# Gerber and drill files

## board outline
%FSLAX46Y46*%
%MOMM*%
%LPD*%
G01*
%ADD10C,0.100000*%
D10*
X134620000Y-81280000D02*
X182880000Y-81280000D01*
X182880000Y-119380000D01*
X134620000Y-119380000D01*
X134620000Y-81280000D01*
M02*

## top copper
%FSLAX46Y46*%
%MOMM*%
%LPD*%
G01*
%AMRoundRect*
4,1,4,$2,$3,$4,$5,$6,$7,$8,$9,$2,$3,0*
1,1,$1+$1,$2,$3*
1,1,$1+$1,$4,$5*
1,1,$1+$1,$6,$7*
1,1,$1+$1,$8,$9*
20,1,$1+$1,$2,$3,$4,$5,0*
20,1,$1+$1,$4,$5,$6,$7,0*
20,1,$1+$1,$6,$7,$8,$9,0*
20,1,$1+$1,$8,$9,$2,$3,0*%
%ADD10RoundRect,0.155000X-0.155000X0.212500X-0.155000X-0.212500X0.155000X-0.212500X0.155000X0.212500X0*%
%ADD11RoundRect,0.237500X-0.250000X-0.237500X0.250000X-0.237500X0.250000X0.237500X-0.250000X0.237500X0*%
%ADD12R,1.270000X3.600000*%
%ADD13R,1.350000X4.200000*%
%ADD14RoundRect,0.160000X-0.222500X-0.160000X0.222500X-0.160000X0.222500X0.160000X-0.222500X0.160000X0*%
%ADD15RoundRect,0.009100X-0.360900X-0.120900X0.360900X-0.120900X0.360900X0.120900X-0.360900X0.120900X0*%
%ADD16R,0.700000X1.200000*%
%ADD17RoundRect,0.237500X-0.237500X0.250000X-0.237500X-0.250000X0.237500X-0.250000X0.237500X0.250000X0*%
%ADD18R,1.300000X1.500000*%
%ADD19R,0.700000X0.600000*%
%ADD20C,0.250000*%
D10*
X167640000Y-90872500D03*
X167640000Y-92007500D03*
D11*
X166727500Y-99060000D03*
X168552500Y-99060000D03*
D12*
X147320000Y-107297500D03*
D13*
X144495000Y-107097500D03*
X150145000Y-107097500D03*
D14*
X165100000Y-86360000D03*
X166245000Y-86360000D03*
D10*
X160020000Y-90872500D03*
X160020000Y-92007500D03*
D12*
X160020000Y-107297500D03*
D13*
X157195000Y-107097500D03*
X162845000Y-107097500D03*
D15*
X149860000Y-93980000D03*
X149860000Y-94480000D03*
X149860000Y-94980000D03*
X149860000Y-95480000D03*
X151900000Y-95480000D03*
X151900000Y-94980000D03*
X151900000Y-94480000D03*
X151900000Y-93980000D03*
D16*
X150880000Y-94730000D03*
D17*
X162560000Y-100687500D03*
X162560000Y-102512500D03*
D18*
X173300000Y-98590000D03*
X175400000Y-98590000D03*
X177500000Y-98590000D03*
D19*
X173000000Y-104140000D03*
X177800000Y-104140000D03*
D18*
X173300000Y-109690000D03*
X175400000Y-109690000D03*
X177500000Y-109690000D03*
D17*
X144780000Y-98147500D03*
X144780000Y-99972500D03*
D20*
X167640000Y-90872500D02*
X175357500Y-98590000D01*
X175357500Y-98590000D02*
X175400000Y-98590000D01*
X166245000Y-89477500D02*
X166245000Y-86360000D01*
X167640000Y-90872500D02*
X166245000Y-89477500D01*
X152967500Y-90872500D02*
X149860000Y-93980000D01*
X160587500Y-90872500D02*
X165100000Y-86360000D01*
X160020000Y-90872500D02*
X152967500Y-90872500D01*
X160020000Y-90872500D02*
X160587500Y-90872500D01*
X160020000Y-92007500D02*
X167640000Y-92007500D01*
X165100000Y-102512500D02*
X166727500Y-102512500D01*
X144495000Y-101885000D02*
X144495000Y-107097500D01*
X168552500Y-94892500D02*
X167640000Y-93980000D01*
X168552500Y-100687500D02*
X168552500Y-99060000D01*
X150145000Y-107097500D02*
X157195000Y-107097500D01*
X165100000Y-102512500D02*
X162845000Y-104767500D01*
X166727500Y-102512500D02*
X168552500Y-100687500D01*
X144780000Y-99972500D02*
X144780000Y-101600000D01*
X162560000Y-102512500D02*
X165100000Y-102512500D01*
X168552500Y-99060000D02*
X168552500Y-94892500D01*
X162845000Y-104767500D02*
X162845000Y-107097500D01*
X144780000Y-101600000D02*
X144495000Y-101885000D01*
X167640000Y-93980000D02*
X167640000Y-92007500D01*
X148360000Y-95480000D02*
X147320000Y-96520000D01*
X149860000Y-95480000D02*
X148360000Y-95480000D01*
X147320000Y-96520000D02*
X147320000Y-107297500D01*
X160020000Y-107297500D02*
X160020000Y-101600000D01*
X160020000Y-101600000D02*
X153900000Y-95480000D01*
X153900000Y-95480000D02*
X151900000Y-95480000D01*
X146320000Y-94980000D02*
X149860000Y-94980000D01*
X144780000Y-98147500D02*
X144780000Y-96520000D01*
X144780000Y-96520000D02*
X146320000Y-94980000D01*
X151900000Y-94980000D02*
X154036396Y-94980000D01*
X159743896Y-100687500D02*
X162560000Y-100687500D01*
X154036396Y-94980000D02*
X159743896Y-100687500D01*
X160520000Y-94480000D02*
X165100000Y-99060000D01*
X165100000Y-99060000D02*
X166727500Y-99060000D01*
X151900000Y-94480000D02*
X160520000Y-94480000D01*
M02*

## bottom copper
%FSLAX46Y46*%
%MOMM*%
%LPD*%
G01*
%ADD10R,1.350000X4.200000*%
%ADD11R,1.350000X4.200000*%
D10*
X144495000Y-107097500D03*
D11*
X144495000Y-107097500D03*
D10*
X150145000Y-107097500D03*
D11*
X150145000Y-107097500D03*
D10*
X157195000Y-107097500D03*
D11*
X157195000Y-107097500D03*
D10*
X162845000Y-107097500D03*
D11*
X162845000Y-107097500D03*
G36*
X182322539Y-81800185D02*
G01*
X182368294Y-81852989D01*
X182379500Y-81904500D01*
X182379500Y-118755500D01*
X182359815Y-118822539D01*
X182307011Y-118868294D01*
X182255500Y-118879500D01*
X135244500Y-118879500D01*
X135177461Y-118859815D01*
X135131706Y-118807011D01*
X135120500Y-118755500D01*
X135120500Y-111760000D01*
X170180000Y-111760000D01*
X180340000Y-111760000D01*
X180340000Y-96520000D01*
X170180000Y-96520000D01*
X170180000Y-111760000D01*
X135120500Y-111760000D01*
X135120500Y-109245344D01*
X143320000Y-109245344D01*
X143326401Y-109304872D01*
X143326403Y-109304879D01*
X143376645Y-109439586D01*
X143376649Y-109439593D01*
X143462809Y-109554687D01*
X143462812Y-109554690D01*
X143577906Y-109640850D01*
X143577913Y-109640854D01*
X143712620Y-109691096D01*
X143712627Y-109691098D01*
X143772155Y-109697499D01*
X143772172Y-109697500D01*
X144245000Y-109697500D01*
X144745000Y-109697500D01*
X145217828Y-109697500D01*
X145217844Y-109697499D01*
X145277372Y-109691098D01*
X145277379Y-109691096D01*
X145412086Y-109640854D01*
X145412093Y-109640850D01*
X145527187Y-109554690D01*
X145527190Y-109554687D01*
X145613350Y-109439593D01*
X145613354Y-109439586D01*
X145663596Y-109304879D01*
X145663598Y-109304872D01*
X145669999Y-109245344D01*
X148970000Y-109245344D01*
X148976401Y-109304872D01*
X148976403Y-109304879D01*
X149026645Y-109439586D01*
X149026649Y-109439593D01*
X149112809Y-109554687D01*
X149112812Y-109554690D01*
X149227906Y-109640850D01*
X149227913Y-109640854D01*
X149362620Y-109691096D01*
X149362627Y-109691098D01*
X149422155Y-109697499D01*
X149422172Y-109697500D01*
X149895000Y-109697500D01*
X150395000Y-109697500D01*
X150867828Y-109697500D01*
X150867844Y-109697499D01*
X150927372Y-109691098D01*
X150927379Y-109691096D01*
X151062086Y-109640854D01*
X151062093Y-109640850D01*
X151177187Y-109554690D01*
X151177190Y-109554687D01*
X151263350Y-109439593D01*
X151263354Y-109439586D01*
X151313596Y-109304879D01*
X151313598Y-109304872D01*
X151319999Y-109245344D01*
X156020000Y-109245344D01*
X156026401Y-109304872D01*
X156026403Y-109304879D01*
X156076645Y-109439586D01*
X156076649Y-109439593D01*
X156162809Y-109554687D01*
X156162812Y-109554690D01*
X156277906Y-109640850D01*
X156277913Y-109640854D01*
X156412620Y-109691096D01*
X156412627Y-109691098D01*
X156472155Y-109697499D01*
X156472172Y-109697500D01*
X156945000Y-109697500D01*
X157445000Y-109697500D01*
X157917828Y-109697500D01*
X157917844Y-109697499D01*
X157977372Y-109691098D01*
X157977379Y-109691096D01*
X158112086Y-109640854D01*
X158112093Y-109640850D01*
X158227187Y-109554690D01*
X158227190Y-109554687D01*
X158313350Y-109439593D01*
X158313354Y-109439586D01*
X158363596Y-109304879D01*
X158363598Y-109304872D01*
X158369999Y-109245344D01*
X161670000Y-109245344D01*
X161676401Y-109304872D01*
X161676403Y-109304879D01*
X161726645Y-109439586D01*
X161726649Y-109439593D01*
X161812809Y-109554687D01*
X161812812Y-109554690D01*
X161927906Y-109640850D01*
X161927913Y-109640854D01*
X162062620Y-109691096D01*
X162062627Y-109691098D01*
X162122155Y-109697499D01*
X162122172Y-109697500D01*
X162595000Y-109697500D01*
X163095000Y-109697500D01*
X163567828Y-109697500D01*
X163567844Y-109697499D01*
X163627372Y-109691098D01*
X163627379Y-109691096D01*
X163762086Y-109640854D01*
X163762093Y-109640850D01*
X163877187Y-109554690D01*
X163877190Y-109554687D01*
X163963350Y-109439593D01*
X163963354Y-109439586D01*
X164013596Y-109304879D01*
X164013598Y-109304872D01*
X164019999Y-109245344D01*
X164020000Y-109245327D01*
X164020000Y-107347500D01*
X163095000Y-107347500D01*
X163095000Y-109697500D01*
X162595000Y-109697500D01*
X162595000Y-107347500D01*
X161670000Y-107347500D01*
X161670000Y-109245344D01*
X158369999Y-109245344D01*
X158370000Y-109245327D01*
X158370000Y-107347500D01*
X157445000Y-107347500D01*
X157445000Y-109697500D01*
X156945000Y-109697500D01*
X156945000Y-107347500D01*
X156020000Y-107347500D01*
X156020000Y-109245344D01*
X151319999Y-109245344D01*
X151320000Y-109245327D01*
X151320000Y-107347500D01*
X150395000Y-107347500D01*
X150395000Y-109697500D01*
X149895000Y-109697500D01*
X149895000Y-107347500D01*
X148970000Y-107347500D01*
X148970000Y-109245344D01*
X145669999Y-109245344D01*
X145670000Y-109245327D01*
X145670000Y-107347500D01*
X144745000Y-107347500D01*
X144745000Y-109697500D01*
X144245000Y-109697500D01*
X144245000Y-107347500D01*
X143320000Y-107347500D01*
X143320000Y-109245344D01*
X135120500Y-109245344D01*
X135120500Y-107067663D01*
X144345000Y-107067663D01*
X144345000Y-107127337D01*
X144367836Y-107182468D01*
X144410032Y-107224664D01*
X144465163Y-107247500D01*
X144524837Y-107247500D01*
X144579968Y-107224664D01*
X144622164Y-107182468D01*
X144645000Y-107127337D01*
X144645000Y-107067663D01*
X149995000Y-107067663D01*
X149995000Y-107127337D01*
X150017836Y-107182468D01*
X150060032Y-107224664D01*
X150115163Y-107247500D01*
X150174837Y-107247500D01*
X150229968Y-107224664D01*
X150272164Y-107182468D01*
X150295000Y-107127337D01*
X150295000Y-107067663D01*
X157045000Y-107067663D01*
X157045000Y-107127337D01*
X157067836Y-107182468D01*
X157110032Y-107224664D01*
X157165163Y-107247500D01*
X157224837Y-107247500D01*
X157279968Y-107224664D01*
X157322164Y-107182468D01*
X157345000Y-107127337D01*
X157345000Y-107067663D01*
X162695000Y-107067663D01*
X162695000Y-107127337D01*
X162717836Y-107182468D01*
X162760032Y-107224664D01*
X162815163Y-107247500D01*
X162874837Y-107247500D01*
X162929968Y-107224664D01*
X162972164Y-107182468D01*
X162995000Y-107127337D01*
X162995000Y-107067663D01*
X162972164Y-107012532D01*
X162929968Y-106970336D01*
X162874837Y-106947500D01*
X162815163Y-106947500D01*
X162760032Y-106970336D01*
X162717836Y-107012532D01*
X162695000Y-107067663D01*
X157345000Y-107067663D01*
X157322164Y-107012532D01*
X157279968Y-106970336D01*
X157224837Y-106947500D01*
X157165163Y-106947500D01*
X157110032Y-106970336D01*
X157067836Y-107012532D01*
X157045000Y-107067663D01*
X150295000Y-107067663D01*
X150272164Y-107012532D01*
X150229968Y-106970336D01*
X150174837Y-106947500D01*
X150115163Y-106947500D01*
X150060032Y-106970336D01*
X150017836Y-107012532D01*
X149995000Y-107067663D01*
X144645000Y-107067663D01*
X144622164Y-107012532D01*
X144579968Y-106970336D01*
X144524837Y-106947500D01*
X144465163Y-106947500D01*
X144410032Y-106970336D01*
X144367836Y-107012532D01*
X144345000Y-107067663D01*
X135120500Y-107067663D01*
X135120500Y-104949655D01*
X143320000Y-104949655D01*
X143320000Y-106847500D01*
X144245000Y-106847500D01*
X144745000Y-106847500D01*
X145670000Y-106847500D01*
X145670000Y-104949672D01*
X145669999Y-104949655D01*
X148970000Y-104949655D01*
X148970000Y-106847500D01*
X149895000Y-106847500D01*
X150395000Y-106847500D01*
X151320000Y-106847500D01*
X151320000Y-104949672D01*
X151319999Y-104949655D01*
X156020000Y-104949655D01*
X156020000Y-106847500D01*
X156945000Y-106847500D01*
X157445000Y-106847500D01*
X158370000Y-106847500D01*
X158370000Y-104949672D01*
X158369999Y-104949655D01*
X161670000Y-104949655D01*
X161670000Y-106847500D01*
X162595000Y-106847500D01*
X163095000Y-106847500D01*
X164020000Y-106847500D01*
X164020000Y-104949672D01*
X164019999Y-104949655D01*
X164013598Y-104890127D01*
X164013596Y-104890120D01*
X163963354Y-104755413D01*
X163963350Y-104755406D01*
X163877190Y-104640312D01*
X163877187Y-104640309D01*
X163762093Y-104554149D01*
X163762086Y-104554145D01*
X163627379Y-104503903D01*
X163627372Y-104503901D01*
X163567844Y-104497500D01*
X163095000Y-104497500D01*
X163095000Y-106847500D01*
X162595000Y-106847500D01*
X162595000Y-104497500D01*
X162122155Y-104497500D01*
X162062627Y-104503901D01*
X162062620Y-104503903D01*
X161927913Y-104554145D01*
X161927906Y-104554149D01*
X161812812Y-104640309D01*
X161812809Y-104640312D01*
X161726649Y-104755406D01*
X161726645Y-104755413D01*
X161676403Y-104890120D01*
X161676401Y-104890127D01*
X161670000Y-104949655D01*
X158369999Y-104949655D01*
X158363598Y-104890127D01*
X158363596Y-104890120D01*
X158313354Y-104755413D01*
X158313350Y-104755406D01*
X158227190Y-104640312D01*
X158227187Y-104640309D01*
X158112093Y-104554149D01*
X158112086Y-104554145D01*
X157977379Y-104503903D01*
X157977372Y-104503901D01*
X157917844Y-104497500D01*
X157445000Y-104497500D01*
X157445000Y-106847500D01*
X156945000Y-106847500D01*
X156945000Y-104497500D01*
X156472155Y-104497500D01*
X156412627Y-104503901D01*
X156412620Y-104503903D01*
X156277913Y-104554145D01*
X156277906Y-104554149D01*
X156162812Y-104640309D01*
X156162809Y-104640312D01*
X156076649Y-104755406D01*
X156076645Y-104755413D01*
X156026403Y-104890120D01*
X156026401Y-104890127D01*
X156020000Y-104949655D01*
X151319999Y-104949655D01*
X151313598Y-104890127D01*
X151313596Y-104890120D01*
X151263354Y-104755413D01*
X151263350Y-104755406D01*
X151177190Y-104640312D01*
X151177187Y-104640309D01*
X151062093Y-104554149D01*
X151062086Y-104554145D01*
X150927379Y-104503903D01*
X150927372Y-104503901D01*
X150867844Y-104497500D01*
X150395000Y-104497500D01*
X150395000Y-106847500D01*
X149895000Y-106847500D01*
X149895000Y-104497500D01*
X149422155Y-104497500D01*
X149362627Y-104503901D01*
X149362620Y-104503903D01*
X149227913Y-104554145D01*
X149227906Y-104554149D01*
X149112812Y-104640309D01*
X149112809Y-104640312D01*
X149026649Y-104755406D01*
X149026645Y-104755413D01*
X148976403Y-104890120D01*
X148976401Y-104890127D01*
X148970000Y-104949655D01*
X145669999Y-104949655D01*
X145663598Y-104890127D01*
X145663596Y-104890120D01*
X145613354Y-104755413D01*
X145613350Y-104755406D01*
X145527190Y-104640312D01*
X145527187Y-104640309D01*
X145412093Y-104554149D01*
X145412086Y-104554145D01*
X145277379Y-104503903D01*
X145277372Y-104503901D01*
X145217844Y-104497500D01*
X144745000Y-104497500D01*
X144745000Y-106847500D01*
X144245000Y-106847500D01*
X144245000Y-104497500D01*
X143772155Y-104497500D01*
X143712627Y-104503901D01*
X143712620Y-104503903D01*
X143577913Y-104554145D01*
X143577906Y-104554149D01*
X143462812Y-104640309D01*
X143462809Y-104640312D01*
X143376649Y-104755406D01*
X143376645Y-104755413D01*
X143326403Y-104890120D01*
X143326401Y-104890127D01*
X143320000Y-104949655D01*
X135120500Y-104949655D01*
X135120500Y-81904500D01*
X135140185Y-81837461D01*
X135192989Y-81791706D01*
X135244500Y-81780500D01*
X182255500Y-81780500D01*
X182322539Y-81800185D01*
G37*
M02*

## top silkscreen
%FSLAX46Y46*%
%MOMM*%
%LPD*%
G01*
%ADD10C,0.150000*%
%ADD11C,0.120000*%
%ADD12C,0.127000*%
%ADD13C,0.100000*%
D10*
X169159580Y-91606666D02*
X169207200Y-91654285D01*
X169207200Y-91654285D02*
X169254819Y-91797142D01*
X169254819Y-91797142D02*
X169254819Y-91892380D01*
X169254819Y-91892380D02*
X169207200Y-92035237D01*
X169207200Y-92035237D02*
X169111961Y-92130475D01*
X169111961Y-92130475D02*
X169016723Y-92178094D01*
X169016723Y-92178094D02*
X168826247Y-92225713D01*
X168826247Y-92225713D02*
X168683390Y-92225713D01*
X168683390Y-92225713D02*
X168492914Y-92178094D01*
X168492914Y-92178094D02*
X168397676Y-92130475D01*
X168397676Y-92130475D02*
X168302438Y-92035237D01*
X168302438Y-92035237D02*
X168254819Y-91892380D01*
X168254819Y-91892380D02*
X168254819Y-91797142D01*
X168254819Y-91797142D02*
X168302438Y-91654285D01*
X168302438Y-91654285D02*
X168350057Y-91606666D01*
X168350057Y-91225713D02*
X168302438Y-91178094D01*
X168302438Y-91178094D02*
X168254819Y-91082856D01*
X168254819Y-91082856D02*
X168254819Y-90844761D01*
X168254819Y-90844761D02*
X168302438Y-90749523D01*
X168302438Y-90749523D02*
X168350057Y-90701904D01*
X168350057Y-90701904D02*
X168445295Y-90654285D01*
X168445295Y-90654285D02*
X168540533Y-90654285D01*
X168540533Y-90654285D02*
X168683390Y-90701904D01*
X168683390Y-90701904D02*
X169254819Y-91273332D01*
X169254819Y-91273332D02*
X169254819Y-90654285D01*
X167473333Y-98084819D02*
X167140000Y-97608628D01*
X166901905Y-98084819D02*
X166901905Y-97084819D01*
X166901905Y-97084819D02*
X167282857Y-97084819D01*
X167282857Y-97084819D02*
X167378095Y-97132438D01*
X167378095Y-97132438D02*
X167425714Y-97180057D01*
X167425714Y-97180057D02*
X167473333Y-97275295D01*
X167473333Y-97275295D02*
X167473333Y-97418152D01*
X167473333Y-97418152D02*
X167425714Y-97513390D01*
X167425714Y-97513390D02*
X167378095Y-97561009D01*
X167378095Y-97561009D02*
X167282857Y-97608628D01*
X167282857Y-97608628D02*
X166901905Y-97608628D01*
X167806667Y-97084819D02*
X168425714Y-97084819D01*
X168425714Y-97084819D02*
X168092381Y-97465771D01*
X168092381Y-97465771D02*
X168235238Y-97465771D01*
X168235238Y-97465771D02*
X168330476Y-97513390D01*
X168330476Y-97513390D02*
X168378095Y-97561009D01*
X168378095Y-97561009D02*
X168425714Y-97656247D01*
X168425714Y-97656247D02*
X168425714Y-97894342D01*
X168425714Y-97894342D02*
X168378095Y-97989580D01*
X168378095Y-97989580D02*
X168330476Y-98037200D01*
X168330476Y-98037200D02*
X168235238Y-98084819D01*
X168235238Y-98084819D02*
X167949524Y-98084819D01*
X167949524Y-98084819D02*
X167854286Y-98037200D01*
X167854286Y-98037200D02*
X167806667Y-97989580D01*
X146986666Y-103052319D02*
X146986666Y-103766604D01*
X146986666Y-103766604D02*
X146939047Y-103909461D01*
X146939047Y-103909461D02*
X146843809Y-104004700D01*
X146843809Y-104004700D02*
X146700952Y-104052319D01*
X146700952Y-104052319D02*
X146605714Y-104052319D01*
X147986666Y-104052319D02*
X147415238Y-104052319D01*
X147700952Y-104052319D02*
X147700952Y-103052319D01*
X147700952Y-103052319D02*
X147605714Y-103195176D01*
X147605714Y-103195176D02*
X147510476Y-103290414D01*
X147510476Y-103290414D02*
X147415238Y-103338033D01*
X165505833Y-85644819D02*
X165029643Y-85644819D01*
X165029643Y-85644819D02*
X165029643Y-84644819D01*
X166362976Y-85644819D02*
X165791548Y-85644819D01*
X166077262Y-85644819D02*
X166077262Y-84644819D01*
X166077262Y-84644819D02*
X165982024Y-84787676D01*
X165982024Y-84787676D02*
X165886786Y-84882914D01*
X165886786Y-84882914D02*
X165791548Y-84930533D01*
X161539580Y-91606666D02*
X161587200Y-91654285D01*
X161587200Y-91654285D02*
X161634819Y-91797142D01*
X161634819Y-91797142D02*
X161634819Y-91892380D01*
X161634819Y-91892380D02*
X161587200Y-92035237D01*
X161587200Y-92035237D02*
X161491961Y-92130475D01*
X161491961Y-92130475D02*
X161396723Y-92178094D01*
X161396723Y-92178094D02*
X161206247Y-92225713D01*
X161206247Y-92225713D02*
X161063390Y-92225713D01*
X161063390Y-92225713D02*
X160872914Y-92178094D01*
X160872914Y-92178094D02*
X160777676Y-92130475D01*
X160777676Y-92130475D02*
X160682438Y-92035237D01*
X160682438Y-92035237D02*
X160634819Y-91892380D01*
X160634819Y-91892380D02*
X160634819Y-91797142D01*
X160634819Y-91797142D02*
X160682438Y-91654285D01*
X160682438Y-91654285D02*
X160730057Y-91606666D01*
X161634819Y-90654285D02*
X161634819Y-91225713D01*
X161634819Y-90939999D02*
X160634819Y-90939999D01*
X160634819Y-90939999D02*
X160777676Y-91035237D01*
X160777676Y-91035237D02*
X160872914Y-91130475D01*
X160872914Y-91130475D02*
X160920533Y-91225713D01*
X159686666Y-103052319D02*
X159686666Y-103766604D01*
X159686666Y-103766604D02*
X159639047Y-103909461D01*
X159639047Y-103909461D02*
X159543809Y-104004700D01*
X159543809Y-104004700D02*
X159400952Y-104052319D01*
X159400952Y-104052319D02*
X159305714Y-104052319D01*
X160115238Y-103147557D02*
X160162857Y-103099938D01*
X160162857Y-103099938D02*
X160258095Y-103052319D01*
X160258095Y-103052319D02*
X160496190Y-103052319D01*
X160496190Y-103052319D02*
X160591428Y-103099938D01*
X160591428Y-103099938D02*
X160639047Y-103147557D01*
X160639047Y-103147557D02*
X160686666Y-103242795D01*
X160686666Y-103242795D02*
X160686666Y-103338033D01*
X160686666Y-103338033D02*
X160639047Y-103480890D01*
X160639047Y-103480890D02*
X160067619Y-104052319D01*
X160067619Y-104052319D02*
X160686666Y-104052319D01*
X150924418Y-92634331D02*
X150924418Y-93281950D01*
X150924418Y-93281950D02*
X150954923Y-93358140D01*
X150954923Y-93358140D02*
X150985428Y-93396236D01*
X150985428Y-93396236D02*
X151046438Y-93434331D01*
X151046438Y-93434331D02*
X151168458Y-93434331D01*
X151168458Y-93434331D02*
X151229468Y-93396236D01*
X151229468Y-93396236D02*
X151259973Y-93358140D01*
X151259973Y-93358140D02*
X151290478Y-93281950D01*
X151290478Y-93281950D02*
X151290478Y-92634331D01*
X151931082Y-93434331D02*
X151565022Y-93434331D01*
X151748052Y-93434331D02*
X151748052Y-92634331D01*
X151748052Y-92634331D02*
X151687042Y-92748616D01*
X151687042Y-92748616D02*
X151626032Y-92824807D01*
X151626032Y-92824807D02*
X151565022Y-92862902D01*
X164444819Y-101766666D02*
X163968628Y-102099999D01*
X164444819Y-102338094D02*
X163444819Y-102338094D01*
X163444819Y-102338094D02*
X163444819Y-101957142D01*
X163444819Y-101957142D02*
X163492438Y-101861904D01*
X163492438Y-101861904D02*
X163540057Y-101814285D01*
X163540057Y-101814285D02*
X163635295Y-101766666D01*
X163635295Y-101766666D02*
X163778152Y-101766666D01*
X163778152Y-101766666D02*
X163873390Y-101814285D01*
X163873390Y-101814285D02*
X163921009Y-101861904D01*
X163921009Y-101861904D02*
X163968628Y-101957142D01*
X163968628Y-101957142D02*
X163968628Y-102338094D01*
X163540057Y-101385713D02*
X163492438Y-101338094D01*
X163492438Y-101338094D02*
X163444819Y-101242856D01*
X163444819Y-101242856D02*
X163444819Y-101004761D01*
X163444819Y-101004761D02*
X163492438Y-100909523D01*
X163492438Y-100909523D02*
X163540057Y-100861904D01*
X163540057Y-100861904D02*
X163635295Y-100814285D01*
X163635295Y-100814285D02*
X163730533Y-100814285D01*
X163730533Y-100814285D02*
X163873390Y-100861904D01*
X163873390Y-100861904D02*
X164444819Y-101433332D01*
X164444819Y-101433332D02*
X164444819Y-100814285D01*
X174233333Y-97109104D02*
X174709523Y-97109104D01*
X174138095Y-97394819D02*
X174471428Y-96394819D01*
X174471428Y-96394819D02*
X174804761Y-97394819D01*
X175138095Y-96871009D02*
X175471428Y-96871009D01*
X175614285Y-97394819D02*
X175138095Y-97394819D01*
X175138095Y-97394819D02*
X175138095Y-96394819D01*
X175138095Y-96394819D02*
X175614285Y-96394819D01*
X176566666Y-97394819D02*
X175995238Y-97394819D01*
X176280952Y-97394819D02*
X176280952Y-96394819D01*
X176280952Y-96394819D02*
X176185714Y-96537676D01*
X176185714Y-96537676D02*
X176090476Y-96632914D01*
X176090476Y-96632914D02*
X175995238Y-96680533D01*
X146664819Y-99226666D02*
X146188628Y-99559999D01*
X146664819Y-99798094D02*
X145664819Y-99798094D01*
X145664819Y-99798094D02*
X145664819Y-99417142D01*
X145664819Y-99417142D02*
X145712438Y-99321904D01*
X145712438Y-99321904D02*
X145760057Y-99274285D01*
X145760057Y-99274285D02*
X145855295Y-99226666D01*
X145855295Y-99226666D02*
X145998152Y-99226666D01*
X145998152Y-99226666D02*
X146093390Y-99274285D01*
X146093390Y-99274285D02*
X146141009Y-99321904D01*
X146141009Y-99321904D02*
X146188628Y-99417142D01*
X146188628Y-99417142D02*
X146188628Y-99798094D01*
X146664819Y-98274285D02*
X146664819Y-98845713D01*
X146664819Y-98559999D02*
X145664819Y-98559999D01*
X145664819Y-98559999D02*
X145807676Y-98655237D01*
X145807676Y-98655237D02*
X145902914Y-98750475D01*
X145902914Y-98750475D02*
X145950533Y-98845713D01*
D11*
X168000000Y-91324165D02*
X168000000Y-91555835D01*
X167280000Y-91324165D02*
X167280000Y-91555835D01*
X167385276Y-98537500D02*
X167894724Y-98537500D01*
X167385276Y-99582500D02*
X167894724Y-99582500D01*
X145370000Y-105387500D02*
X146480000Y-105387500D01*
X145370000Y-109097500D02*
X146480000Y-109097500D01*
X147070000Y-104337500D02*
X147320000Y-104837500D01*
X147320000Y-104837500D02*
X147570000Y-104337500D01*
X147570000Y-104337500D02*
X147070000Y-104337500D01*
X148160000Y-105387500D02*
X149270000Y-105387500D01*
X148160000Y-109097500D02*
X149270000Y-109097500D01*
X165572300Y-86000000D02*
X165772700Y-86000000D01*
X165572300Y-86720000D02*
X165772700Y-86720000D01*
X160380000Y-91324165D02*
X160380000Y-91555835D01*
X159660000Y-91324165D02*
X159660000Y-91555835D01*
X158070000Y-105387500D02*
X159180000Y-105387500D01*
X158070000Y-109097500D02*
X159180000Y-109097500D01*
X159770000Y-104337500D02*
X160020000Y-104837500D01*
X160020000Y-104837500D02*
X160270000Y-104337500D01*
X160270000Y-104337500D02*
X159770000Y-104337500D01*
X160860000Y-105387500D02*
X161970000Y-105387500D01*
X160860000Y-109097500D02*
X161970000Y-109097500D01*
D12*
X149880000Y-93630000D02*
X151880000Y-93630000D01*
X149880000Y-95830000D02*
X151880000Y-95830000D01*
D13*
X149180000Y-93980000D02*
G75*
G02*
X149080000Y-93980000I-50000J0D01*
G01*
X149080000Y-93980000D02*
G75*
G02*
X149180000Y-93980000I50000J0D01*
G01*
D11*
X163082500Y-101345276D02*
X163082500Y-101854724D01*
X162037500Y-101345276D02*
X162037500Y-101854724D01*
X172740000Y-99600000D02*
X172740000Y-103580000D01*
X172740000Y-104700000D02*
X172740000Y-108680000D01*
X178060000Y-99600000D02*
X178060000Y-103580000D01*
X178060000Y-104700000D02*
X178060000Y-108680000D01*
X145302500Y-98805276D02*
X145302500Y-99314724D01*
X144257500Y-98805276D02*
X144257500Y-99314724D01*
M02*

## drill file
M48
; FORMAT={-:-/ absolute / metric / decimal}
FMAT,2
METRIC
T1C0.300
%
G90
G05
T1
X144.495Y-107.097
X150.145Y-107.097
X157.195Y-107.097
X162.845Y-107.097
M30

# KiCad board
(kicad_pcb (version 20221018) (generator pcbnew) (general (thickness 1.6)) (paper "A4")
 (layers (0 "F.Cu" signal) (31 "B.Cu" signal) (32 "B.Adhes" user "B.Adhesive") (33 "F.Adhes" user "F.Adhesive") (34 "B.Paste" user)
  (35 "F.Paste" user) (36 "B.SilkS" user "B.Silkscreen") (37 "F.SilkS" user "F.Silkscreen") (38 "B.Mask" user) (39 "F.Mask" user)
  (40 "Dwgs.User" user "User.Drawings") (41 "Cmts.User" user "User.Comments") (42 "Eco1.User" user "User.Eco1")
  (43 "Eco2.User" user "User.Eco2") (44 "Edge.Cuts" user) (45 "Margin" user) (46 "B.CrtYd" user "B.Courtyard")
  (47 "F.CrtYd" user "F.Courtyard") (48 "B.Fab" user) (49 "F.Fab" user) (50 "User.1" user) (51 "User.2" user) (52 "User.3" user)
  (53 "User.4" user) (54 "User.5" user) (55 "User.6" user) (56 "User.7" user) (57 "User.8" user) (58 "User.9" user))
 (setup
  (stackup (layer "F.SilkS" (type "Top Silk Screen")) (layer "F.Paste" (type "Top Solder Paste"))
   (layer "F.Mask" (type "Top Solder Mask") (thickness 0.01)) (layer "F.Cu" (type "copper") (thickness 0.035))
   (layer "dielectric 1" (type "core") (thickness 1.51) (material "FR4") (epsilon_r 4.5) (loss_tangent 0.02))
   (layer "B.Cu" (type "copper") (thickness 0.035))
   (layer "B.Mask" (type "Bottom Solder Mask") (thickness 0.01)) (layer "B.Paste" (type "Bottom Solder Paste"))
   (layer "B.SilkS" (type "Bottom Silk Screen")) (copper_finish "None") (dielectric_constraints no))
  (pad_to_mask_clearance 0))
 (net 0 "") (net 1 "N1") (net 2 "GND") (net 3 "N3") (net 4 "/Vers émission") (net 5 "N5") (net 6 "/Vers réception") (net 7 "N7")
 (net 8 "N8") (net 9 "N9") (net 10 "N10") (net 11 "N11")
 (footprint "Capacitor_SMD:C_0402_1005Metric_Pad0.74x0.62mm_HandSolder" (layer "F.Cu") (at 167.64 91.44 -90)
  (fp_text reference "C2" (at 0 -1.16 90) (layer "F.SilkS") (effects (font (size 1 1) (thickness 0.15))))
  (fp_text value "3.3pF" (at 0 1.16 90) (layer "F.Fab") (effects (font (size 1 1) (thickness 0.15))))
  (fp_line (start -0.115835 -0.36) (end 0.115835 -0.36) (stroke (width 0.12) (type solid)) (layer "F.SilkS"))
  (fp_line (start -0.115835 0.36) (end 0.115835 0.36) (stroke (width 0.12) (type solid)) (layer "F.SilkS"))
  (pad "1" smd roundrect (at -0.5675 0 270) (size 0.735 0.62) (layers "F.Cu" "F.Paste" "F.Mask") (roundrect_rratio 0.25) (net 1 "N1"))
  (pad "2" smd roundrect (at 0.5675 0 270) (size 0.735 0.62) (layers "F.Cu" "F.Paste" "F.Mask") (roundrect_rratio 0.25) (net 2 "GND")))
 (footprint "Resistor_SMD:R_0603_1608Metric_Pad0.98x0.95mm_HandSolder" (layer "F.Cu") (at 167.64 99.06)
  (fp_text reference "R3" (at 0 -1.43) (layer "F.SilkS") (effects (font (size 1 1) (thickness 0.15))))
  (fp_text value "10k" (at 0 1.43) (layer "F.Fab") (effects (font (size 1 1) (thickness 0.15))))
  (fp_line (start -0.254724 -0.5225) (end 0.254724 -0.5225) (stroke (width 0.12) (type solid)) (layer "F.SilkS"))
  (fp_line (start -0.254724 0.5225) (end 0.254724 0.5225) (stroke (width 0.12) (type solid)) (layer "F.SilkS"))
  (pad "1" smd roundrect (at -0.9125 0) (size 0.975 0.95) (layers "F.Cu" "F.Paste" "F.Mask") (roundrect_rratio 0.25) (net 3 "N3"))
  (pad "2" smd roundrect (at 0.9125 0) (size 0.975 0.95) (layers "F.Cu" "F.Paste" "F.Mask") (roundrect_rratio 0.25) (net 2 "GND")))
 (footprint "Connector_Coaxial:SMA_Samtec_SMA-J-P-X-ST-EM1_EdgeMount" (layer "F.Cu") (at 147.32 107.0975)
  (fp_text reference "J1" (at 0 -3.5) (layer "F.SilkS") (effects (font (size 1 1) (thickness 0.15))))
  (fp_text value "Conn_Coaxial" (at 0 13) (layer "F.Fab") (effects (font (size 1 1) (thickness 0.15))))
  (fp_line (start -1.95 -1.71) (end -0.84 -1.71) (stroke (width 0.12) (type solid)) (layer "F.SilkS"))
  (fp_line (start -1.95 2) (end -0.84 2) (stroke (width 0.12) (type solid)) (layer "F.SilkS"))
  (fp_line (start -0.25 -2.76) (end 0 -2.26) (stroke (width 0.12) (type solid)) (layer "F.SilkS"))
  (fp_line (start 0 -2.26) (end 0.25 -2.76) (stroke (width 0.12) (type solid)) (layer "F.SilkS"))
  (fp_line (start 0.25 -2.76) (end -0.25 -2.76) (stroke (width 0.12) (type solid)) (layer "F.SilkS"))
  (fp_line (start 0.84 -1.71) (end 1.95 -1.71) (stroke (width 0.12) (type solid)) (layer "F.SilkS"))
  (fp_line (start 0.84 2) (end 1.95 2) (stroke (width 0.12) (type solid)) (layer "F.SilkS"))
  (pad "1" smd rect (at 0 0.2) (size 1.27 3.6) (layers "F.Cu" "F.Paste" "F.Mask") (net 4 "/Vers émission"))
  (pad "2" thru_hole rect (at -2.825 0) (size 1.35 4.2) (drill 0.3) (layers "*.Cu" "*.Mask") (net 2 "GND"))
  (pad "2" smd rect (at -2.825 0) (size 1.35 4.2) (layers "B.Cu" "B.Paste" "B.Mask") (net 2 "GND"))
  (pad "2" thru_hole rect (at 2.825 0) (size 1.35 4.2) (drill 0.3) (layers "*.Cu" "*.Mask") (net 2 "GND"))
  (pad "2" smd rect (at 2.825 0) (size 1.35 4.2) (layers "B.Cu" "B.Paste" "B.Mask") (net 2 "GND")))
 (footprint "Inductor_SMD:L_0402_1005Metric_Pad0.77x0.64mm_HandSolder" (layer "F.Cu") (at 165.6725 86.36)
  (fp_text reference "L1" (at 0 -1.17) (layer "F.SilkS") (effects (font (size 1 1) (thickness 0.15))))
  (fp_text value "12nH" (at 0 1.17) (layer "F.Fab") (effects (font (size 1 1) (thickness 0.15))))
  (fp_line (start -0.1002 -0.36) (end 0.1002 -0.36) (stroke (width 0.12) (type solid)) (layer "F.SilkS"))
  (fp_line (start -0.1002 0.36) (end 0.1002 0.36) (stroke (width 0.12) (type solid)) (layer "F.SilkS"))
  (pad "1" smd roundrect (at -0.5725 0) (size 0.765 0.64) (layers "F.Cu" "F.Paste" "F.Mask") (roundrect_rratio 0.25) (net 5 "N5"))
  (pad "2" smd roundrect (at 0.5725 0) (size 0.765 0.64) (layers "F.Cu" "F.Paste" "F.Mask") (roundrect_rratio 0.25) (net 1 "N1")))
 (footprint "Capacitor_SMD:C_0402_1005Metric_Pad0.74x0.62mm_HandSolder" (layer "F.Cu") (at 160.02 91.44 -90)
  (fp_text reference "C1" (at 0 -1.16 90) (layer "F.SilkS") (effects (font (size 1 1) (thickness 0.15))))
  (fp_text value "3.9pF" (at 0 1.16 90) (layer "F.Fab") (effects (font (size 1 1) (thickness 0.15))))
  (fp_line (start -0.115835 -0.36) (end 0.115835 -0.36) (stroke (width 0.12) (type solid)) (layer "F.SilkS"))
  (fp_line (start -0.115835 0.36) (end 0.115835 0.36) (stroke (width 0.12) (type solid)) (layer "F.SilkS"))
  (pad "1" smd roundrect (at -0.5675 0 270) (size 0.735 0.62) (layers "F.Cu" "F.Paste" "F.Mask") (roundrect_rratio 0.25) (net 5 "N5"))
  (pad "2" smd roundrect (at 0.5675 0 270) (size 0.735 0.62) (layers "F.Cu" "F.Paste" "F.Mask") (roundrect_rratio 0.25) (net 2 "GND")))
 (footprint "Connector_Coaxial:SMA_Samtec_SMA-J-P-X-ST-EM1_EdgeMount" (layer "F.Cu") (at 160.02 107.0975)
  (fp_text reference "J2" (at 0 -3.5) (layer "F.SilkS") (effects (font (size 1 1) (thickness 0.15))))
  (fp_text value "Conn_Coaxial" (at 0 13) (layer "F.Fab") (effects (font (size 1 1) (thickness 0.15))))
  (fp_line (start -1.95 -1.71) (end -0.84 -1.71) (stroke (width 0.12) (type solid)) (layer "F.SilkS"))
  (fp_line (start -1.95 2) (end -0.84 2) (stroke (width 0.12) (type solid)) (layer "F.SilkS"))
  (fp_line (start -0.25 -2.76) (end 0 -2.26) (stroke (width 0.12) (type solid)) (layer "F.SilkS"))
  (fp_line (start 0 -2.26) (end 0.25 -2.76) (stroke (width 0.12) (type solid)) (layer "F.SilkS"))
  (fp_line (start 0.25 -2.76) (end -0.25 -2.76) (stroke (width 0.12) (type solid)) (layer "F.SilkS"))
  (fp_line (start 0.84 -1.71) (end 1.95 -1.71) (stroke (width 0.12) (type solid)) (layer "F.SilkS"))
  (fp_line (start 0.84 2) (end 1.95 2) (stroke (width 0.12) (type solid)) (layer "F.SilkS"))
  (pad "1" smd rect (at 0 0.2) (size 1.27 3.6) (layers "F.Cu" "F.Paste" "F.Mask") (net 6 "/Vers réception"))
  (pad "2" thru_hole rect (at -2.825 0) (size 1.35 4.2) (drill 0.3) (layers "*.Cu" "*.Mask") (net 2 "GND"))
  (pad "2" smd rect (at -2.825 0) (size 1.35 4.2) (layers "B.Cu" "B.Paste" "B.Mask") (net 2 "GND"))
  (pad "2" thru_hole rect (at 2.825 0) (size 1.35 4.2) (drill 0.3) (layers "*.Cu" "*.Mask") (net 2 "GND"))
  (pad "2" smd rect (at 2.825 0) (size 1.35 4.2) (layers "B.Cu" "B.Paste" "B.Mask") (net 2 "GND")))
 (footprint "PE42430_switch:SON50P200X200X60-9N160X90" (layer "F.Cu") (at 150.88 94.73)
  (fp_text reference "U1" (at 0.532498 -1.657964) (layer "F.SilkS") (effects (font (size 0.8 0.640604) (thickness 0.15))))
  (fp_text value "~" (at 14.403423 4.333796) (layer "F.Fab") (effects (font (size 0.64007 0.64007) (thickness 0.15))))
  (fp_line (start -1 -1.1) (end 1 -1.1) (stroke (width 0.127) (type solid)) (layer "F.SilkS"))
  (fp_line (start -1 1.1) (end 1 1.1) (stroke (width 0.127) (type solid)) (layer "F.SilkS"))
  (fp_circle (center -1.75 -0.75) (end -1.7 -0.75) (stroke (width 0.1) (type solid)) (fill none) (layer "F.SilkS"))
  (pad "1" smd roundrect (at -1.02 -0.75) (size 0.74 0.26) (layers "F.Cu" "F.Paste" "F.Mask") (roundrect_rratio 0.035) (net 5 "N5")
   (solder_mask_margin 0.102))
  (pad "2" smd roundrect (at -1.02 -0.25) (size 0.74 0.26) (layers "F.Cu" "F.Paste" "F.Mask") (roundrect_rratio 0.035) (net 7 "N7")
   (solder_mask_margin 0.102))
  (pad "3" smd roundrect (at -1.02 0.25) (size 0.74 0.26) (layers "F.Cu" "F.Paste" "F.Mask") (roundrect_rratio 0.035) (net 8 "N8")
   (solder_mask_margin 0.102))
  (pad "4" smd roundrect (at -1.02 0.75) (size 0.74 0.26) (layers "F.Cu" "F.Paste" "F.Mask") (roundrect_rratio 0.035)
   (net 4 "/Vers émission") (solder_mask_margin 0.102))
  (pad "5" smd roundrect (at 1.02 0.75) (size 0.74 0.26) (layers "F.Cu" "F.Paste" "F.Mask") (roundrect_rratio 0.035)
   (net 6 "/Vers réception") (solder_mask_margin 0.102))
  (pad "6" smd roundrect (at 1.02 0.25) (size 0.74 0.26) (layers "F.Cu" "F.Paste" "F.Mask") (roundrect_rratio 0.035) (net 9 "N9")
   (solder_mask_margin 0.102))
  (pad "7" smd roundrect (at 1.02 -0.25) (size 0.74 0.26) (layers "F.Cu" "F.Paste" "F.Mask") (roundrect_rratio 0.035) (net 3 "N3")
   (solder_mask_margin 0.102))
  (pad "8" smd roundrect (at 1.02 -0.75) (size 0.74 0.26) (layers "F.Cu" "F.Paste" "F.Mask") (roundrect_rratio 0.035) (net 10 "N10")
   (solder_mask_margin 0.102))
  (pad "EP" smd rect (at 0 0) (size 0.7 1.2) (layers "F.Cu" "F.Mask") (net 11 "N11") (solder_mask_margin 0.102)))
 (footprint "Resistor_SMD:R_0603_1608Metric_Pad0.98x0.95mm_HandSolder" (layer "F.Cu") (at 162.56 101.6 -90)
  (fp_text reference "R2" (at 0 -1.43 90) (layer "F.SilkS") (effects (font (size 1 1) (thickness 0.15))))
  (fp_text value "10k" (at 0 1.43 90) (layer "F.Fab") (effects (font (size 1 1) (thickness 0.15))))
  (fp_line (start -0.254724 -0.5225) (end 0.254724 -0.5225) (stroke (width 0.12) (type solid)) (layer "F.SilkS"))
  (fp_line (start -0.254724 0.5225) (end 0.254724 0.5225) (stroke (width 0.12) (type solid)) (layer "F.SilkS"))
  (pad "1" smd roundrect (at -0.9125 0 270) (size 0.975 0.95) (layers "F.Cu" "F.Paste" "F.Mask") (roundrect_rratio 0.25) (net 9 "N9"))
  (pad "2" smd roundrect (at 0.9125 0 270) (size 0.975 0.95) (layers "F.Cu" "F.Paste" "F.Mask") (roundrect_rratio 0.25) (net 2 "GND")))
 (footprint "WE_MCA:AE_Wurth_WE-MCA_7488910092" (layer "F.Cu") (at 175.4 104.14)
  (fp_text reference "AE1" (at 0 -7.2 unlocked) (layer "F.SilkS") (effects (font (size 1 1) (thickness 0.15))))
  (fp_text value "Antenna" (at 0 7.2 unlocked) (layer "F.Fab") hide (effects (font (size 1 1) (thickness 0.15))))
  (fp_line (start -2.66 -4.54) (end -2.66 -0.56) (stroke (width 0.12) (type default)) (layer "F.SilkS"))
  (fp_line (start -2.66 0.56) (end -2.66 4.54) (stroke (width 0.12) (type default)) (layer "F.SilkS"))
  (fp_line (start 2.66 -4.54) (end 2.66 -0.56) (stroke (width 0.12) (type default)) (layer "F.SilkS"))
  (fp_line (start 2.66 0.56) (end 2.66 4.54) (stroke (width 0.12) (type default)) (layer "F.SilkS"))
  (pad "1" smd rect (at -2.1 -5.55) (size 1.3 1.5) (layers "F.Cu" "F.Paste" "F.Mask"))
  (pad "2" smd rect (at 0 -5.55) (size 1.3 1.5) (layers "F.Cu" "F.Paste" "F.Mask") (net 1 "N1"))
  (pad "3" smd rect (at 2.1 -5.55) (size 1.3 1.5) (layers "F.Cu" "F.Paste" "F.Mask"))
  (pad "4" smd rect (at -2.4 0) (size 0.7 0.6) (layers "F.Cu" "F.Paste" "F.Mask"))
  (pad "5" smd rect (at 2.4 0) (size 0.7 0.6) (layers "F.Cu" "F.Paste" "F.Mask"))
  (pad "6" smd rect (at -2.1 5.55) (size 1.3 1.5) (layers "F.Cu" "F.Paste" "F.Mask"))
  (pad "7" smd rect (at 0 5.55) (size 1.3 1.5) (layers "F.Cu" "F.Paste" "F.Mask"))
  (pad "8" smd rect (at 2.1 5.55) (size 1.3 1.5) (layers "F.Cu" "F.Paste" "F.Mask")))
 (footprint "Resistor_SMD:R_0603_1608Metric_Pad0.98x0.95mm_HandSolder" (layer "F.Cu") (at 144.78 99.06 -90)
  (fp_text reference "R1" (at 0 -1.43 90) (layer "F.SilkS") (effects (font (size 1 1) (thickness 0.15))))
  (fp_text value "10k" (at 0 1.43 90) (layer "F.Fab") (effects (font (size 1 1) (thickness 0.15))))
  (fp_line (start -0.254724 -0.5225) (end 0.254724 -0.5225) (stroke (width 0.12) (type solid)) (layer "F.SilkS"))
  (fp_line (start -0.254724 0.5225) (end 0.254724 0.5225) (stroke (width 0.12) (type solid)) (layer "F.SilkS"))
  (pad "1" smd roundrect (at -0.9125 0 270) (size 0.975 0.95) (layers "F.Cu" "F.Paste" "F.Mask") (roundrect_rratio 0.25) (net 8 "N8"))
  (pad "2" smd roundrect (at 0.9125 0 270) (size 0.975 0.95) (layers "F.Cu" "F.Paste" "F.Mask") (roundrect_rratio 0.25) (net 2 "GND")))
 (gr_rect (start 134.62 81.28) (end 182.88 119.38) (stroke (width 0.1) (type default)) (fill none) (layer "Edge.Cuts"))
 (segment (start 167.64 90.8725) (end 175.3575 98.59) (width 0.25) (layer "F.Cu") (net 1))
 (segment (start 175.3575 98.59) (end 175.4 98.59) (width 0.25) (layer "F.Cu") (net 1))
 (segment (start 166.245 89.4775) (end 166.245 86.36) (width 0.25) (layer "F.Cu") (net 1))
 (segment (start 167.64 90.8725) (end 166.245 89.4775) (width 0.25) (layer "F.Cu") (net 1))
 (segment (start 152.9675 90.8725) (end 149.86 93.98) (width 0.25) (layer "F.Cu") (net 5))
 (segment (start 160.5875 90.8725) (end 165.1 86.36) (width 0.25) (layer "F.Cu") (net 5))
 (segment (start 160.02 90.8725) (end 152.9675 90.8725) (width 0.25) (layer "F.Cu") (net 5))
 (segment (start 160.02 90.8725) (end 160.5875 90.8725) (width 0.25) (layer "F.Cu") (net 5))
 (segment (start 160.02 92.0075) (end 167.64 92.0075) (width 0.25) (layer "F.Cu") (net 2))
 (segment (start 165.1 102.5125) (end 166.7275 102.5125) (width 0.25) (layer "F.Cu") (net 2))
 (segment (start 144.495 101.885) (end 144.495 107.0975) (width 0.25) (layer "F.Cu") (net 2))
 (segment (start 168.5525 94.8925) (end 167.64 93.98) (width 0.25) (layer "F.Cu") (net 2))
 (segment (start 168.5525 100.6875) (end 168.5525 99.06) (width 0.25) (layer "F.Cu") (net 2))
 (segment (start 150.145 107.0975) (end 157.195 107.0975) (width 0.25) (layer "F.Cu") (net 2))
 (segment (start 165.1 102.5125) (end 162.845 104.7675) (width 0.25) (layer "F.Cu") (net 2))
 (segment (start 166.7275 102.5125) (end 168.5525 100.6875) (width 0.25) (layer "F.Cu") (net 2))
 (segment (start 144.78 99.9725) (end 144.78 101.6) (width 0.25) (layer "F.Cu") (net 2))
 (segment (start 162.56 102.5125) (end 165.1 102.5125) (width 0.25) (layer "F.Cu") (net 2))
 (segment (start 168.5525 99.06) (end 168.5525 94.8925) (width 0.25) (layer "F.Cu") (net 2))
 (segment (start 162.845 104.7675) (end 162.845 107.0975) (width 0.25) (layer "F.Cu") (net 2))
 (segment (start 144.78 101.6) (end 144.495 101.885) (width 0.25) (layer "F.Cu") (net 2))
 (segment (start 167.64 93.98) (end 167.64 92.0075) (width 0.25) (layer "F.Cu") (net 2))
 (segment (start 148.36 95.48) (end 147.32 96.52) (width 0.25) (layer "F.Cu") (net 4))
 (segment (start 149.86 95.48) (end 148.36 95.48) (width 0.25) (layer "F.Cu") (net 4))
 (segment (start 147.32 96.52) (end 147.32 107.2975) (width 0.25) (layer "F.Cu") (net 4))
 (segment (start 160.02 107.2975) (end 160.02 101.6) (width 0.25) (layer "F.Cu") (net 6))
 (segment (start 160.02 101.6) (end 153.9 95.48) (width 0.25) (layer "F.Cu") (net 6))
 (segment (start 153.9 95.48) (end 151.9 95.48) (width 0.25) (layer "F.Cu") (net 6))
 (segment (start 146.32 94.98) (end 149.86 94.98) (width 0.25) (layer "F.Cu") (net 8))
 (segment (start 144.78 98.1475) (end 144.78 96.52) (width 0.25) (layer "F.Cu") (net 8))
 (segment (start 144.78 96.52) (end 146.32 94.98) (width 0.25) (layer "F.Cu") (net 8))
 (segment (start 151.9 94.98) (end 154.036396 94.98) (width 0.25) (layer "F.Cu") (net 9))
 (segment (start 159.743896 100.6875) (end 162.56 100.6875) (width 0.25) (layer "F.Cu") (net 9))
 (segment (start 154.036396 94.98) (end 159.743896 100.6875) (width 0.25) (layer "F.Cu") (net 9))
 (segment (start 160.52 94.48) (end 165.1 99.06) (width 0.25) (layer "F.Cu") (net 3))
 (segment (start 165.1 99.06) (end 166.7275 99.06) (width 0.25) (layer "F.Cu") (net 3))
 (segment (start 151.9 94.48) (end 160.52 94.48) (width 0.25) (layer "F.Cu") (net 3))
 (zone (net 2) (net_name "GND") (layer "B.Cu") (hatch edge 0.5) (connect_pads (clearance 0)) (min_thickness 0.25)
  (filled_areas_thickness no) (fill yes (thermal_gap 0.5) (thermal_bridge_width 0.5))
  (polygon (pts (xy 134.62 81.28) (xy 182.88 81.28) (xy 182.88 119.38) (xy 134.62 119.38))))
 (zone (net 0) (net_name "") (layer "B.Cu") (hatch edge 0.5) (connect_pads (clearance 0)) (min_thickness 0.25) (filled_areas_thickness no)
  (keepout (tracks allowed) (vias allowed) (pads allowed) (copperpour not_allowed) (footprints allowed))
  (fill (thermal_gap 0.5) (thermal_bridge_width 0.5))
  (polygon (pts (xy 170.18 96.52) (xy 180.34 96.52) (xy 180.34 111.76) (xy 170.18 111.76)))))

